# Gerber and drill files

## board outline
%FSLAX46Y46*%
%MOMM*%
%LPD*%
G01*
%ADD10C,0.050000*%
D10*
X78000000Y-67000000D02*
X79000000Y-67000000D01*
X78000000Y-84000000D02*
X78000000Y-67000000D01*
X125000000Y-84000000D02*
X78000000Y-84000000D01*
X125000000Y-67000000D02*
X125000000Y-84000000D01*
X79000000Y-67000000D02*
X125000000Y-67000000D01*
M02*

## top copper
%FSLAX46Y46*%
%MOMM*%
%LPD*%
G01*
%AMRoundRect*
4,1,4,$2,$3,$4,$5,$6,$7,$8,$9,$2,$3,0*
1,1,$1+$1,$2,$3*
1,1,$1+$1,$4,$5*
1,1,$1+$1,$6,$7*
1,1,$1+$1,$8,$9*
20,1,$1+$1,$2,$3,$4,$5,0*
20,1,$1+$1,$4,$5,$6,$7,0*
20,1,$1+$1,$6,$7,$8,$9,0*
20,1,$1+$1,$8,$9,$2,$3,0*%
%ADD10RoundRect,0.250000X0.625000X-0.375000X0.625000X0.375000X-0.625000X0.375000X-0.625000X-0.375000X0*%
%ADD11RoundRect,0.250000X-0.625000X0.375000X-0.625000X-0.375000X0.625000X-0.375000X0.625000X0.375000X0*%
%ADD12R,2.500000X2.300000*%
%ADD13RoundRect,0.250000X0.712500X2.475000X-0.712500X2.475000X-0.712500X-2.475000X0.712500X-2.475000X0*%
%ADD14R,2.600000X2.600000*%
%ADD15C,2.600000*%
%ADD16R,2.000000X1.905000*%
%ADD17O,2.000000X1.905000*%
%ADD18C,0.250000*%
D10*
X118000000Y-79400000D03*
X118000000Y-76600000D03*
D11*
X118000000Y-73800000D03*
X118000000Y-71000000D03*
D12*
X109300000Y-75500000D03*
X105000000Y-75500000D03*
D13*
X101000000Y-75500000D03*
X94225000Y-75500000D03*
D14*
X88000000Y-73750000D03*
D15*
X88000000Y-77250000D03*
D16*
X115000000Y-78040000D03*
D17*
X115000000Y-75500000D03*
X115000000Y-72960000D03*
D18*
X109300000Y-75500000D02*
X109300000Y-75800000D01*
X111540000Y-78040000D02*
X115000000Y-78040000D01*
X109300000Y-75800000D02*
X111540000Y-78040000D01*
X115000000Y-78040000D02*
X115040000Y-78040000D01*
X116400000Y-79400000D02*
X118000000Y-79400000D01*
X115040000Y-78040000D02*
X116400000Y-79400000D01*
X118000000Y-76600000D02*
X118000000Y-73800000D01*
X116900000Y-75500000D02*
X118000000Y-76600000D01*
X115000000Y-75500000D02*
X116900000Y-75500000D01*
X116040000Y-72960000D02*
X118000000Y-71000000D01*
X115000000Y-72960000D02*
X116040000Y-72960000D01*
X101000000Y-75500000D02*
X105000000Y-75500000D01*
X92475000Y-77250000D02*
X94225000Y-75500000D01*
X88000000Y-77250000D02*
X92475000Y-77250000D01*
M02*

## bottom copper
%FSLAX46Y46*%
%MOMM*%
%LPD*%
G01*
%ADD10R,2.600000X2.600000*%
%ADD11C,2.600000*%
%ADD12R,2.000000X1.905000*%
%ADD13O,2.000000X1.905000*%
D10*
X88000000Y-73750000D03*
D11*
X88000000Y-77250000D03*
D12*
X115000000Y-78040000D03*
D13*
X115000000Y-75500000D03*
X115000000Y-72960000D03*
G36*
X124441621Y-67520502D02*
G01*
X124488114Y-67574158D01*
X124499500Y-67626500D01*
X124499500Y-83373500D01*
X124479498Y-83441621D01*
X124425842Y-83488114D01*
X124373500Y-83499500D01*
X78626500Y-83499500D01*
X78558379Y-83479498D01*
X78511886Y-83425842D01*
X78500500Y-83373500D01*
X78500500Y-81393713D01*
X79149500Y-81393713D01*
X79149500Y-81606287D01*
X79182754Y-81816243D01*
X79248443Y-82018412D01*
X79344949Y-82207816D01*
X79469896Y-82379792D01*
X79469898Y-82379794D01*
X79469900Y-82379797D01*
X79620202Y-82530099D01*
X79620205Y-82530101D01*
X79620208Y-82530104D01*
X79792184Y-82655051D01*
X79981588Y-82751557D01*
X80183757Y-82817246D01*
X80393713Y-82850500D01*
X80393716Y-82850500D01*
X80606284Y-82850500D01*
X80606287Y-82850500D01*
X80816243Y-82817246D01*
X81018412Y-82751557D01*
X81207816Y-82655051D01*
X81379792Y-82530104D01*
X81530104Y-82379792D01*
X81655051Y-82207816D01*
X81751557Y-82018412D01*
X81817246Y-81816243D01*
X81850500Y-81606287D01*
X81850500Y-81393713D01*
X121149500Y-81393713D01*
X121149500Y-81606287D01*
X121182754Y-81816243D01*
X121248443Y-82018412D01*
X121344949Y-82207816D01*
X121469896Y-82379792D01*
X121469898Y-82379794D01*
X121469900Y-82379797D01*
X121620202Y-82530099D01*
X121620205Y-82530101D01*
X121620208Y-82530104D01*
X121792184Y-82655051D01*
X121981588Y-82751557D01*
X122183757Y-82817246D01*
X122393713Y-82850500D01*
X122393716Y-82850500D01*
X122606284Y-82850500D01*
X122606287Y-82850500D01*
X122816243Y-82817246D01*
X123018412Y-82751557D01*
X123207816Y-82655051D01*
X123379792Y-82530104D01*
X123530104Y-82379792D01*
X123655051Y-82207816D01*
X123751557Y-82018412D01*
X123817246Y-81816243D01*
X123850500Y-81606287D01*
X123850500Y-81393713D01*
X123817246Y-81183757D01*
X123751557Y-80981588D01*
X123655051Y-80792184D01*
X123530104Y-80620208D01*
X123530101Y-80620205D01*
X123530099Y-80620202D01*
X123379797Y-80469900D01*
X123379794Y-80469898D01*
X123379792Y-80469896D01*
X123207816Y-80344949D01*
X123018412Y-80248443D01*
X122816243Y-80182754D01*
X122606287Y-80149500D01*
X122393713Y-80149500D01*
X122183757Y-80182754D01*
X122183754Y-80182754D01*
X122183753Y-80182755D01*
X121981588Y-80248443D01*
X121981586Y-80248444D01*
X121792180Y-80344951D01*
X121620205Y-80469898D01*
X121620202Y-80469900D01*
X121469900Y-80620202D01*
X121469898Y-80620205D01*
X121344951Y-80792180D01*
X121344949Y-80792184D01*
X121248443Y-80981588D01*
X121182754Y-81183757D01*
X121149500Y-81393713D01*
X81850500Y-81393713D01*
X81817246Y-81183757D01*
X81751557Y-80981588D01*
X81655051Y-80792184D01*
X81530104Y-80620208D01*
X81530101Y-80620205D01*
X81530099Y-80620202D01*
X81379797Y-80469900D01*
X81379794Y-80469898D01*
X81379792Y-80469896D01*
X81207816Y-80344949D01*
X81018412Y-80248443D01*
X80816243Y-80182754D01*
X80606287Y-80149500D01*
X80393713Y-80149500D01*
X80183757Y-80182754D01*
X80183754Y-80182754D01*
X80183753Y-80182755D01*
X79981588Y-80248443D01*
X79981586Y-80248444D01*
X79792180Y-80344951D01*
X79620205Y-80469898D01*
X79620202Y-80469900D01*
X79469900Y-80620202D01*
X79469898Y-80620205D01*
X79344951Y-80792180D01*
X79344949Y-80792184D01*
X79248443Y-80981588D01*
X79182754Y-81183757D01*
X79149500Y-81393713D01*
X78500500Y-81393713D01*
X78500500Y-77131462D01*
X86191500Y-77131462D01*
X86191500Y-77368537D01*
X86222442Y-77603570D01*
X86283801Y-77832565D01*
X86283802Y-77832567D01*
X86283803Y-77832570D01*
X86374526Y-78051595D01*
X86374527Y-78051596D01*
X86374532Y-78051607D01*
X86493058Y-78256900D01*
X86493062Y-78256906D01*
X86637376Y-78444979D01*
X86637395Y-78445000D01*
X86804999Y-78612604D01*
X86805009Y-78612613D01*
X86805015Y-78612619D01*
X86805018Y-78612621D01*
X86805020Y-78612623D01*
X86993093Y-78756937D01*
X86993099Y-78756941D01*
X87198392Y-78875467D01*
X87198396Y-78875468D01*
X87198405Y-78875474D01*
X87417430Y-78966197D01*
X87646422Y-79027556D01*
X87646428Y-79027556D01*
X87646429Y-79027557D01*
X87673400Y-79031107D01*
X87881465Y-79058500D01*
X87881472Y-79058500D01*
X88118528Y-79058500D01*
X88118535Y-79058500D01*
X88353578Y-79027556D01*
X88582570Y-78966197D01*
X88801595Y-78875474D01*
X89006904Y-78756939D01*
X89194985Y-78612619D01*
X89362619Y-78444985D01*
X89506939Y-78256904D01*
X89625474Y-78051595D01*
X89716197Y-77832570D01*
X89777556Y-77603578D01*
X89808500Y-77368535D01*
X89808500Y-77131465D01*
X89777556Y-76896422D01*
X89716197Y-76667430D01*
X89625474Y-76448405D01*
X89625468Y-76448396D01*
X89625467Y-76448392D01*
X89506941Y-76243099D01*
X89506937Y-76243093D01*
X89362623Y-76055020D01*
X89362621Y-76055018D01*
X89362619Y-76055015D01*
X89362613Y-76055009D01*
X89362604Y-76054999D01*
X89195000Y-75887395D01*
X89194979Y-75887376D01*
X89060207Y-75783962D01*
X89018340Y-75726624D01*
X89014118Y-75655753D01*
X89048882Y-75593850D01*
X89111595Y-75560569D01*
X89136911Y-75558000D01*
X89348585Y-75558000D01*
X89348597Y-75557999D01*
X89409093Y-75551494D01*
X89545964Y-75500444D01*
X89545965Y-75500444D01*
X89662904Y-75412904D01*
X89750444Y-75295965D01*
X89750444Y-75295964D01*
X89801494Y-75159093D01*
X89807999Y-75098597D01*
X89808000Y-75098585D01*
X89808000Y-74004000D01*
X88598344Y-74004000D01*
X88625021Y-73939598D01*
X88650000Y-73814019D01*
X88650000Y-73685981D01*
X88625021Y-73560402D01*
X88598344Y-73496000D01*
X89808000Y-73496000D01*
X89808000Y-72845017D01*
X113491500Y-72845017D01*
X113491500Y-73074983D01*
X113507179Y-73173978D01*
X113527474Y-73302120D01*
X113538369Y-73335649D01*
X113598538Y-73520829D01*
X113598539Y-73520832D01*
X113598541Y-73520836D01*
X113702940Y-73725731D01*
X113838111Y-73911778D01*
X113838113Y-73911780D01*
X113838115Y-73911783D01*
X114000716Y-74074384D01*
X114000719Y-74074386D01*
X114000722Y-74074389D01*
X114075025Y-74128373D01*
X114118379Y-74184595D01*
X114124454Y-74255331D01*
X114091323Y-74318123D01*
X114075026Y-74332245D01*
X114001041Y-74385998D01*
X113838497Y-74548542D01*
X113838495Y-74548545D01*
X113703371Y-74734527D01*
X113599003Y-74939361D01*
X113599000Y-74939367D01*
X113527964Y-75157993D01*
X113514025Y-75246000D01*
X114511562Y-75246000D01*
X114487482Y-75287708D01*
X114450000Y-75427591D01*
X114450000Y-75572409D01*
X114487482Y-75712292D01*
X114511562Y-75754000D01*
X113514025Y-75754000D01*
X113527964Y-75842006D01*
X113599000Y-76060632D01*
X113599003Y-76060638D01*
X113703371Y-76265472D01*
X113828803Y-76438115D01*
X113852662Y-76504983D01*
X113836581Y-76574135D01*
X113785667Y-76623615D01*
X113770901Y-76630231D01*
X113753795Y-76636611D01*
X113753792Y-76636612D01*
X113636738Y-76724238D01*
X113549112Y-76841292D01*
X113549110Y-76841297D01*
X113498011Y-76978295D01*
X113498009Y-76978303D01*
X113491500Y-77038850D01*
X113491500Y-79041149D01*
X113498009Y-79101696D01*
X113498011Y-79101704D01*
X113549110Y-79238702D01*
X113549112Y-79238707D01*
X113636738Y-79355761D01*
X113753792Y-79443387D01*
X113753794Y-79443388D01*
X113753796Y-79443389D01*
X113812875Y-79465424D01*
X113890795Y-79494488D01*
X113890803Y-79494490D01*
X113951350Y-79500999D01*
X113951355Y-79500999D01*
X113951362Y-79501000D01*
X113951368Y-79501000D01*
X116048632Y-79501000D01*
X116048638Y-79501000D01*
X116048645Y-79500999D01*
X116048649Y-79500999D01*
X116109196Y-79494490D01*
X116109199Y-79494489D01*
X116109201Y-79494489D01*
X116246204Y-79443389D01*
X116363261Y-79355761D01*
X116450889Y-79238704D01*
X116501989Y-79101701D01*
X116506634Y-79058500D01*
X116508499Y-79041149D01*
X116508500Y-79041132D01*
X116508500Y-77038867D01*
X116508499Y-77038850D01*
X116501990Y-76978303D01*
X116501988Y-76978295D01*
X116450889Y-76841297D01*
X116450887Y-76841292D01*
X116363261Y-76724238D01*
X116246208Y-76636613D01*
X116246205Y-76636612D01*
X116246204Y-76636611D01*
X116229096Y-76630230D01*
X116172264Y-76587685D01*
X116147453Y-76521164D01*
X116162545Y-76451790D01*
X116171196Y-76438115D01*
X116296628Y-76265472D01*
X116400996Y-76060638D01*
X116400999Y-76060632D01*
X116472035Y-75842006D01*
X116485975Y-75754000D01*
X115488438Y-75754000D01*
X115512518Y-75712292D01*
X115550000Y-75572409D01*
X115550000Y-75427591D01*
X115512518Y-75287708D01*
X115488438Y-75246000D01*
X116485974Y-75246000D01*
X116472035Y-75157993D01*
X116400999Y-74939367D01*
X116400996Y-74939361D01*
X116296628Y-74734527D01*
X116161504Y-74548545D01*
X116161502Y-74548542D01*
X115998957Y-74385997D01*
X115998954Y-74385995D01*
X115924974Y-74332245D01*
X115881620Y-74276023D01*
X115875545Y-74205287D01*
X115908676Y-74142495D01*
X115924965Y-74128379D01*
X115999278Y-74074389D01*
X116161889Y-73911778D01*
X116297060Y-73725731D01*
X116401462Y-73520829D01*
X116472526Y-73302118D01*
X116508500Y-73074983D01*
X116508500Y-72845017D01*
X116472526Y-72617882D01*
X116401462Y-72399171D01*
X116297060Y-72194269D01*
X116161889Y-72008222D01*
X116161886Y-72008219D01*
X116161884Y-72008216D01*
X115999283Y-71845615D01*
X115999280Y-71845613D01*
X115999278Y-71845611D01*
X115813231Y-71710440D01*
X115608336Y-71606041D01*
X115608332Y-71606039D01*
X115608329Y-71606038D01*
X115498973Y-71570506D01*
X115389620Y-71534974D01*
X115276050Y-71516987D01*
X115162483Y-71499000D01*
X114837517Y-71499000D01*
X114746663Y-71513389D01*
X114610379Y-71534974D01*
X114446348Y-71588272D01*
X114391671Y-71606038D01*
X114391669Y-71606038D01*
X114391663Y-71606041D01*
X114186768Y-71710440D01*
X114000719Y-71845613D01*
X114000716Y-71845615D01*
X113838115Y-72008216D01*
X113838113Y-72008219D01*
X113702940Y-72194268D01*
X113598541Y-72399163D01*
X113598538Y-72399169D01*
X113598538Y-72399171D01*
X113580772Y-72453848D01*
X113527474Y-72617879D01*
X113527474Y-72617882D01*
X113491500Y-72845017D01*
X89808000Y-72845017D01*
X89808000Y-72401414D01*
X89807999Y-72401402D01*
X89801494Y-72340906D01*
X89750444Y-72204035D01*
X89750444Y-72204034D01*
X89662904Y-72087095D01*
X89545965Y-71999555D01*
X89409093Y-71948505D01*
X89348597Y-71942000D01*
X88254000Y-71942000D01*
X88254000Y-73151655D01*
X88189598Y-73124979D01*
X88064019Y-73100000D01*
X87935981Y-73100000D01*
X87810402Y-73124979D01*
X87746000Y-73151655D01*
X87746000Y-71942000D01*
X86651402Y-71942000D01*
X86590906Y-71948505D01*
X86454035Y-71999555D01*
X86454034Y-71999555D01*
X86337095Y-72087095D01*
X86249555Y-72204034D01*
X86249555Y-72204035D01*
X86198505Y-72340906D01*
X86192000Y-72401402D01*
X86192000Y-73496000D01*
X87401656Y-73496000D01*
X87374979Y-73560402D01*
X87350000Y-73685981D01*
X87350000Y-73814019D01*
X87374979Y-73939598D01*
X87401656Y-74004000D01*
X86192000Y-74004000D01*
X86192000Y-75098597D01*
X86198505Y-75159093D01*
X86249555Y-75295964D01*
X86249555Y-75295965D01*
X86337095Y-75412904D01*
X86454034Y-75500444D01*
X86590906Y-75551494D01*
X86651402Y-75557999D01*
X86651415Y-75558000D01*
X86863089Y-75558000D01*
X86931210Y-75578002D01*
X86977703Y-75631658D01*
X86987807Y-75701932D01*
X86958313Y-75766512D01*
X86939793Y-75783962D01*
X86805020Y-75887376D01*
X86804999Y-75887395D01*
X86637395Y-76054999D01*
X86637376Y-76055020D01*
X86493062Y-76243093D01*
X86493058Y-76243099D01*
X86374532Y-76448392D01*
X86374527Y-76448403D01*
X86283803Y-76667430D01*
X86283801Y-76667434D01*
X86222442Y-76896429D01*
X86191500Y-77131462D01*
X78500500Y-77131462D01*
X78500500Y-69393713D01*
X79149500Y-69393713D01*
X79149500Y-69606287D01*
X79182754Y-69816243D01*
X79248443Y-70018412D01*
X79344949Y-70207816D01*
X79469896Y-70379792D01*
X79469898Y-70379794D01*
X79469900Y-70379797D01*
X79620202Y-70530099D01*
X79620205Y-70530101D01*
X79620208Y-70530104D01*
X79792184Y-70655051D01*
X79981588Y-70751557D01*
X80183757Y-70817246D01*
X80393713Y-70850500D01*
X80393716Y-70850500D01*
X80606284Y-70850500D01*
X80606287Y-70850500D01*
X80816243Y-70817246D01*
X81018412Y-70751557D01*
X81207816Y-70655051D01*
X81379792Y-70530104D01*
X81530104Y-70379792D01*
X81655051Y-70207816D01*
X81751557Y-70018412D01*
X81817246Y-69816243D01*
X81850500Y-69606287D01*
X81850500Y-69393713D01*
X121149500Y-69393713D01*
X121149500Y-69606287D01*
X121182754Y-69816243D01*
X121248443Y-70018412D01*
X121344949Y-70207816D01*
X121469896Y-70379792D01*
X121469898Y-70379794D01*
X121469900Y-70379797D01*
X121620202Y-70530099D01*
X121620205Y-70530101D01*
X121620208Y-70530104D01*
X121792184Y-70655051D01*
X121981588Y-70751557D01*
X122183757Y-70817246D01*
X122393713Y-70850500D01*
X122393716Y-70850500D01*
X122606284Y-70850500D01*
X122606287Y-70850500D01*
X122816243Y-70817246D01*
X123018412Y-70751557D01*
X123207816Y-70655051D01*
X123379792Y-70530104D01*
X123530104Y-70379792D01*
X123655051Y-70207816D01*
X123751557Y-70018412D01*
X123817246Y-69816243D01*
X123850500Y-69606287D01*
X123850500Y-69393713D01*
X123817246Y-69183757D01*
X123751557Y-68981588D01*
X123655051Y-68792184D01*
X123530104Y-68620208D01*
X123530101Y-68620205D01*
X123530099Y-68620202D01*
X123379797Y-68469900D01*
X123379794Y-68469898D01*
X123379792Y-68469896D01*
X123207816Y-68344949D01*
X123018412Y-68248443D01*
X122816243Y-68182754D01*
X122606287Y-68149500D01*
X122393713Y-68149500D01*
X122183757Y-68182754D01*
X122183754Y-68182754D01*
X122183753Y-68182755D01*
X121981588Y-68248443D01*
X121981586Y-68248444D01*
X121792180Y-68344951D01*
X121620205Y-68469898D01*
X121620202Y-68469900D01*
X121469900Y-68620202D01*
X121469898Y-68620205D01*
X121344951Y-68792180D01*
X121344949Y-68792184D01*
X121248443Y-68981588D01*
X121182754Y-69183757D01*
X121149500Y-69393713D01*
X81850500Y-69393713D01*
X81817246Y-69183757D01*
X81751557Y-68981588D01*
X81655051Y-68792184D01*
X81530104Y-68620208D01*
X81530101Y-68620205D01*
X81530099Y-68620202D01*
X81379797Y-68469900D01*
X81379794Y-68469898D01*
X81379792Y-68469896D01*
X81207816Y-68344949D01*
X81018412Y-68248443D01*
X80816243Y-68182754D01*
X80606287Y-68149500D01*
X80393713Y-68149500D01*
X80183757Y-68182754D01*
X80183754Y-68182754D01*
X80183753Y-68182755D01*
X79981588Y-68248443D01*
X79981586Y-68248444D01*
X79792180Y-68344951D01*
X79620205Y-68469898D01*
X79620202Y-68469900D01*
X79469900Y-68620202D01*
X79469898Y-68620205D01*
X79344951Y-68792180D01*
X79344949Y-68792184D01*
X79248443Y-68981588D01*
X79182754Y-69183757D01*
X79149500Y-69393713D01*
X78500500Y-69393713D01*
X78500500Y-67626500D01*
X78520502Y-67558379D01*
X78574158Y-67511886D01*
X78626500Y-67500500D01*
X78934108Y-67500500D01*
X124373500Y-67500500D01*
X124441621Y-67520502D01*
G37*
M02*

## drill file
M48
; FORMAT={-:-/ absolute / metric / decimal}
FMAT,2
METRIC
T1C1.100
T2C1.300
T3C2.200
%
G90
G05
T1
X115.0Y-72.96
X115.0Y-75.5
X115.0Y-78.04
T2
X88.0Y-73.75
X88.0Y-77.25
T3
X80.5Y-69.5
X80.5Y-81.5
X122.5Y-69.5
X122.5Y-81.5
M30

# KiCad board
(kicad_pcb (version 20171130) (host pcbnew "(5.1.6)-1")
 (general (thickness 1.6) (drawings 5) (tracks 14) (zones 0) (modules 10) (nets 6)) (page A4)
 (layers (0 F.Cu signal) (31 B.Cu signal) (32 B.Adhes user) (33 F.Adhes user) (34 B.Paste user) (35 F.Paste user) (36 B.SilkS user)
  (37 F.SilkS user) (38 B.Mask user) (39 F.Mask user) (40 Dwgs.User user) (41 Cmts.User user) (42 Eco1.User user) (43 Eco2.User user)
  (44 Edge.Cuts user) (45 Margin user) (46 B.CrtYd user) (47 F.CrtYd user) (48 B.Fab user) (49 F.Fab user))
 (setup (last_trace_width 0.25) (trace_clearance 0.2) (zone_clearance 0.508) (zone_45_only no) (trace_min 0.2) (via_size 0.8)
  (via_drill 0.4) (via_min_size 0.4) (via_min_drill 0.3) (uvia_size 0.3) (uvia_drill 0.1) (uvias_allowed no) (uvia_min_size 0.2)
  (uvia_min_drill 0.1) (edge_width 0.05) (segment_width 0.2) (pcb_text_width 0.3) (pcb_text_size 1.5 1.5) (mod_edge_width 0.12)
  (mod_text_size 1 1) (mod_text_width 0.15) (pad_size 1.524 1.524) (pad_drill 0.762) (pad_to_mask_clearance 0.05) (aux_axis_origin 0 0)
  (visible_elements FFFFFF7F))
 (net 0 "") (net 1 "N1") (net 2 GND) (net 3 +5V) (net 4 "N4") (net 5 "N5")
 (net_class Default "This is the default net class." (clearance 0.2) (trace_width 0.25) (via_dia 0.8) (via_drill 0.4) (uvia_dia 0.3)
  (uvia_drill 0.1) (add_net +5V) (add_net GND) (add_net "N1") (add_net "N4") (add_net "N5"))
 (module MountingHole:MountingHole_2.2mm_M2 (layer F.Cu) (at 80.5 69.5)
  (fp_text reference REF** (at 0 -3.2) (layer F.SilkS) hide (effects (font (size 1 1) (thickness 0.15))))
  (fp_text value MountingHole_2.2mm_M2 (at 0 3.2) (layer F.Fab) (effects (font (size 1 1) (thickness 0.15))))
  (pad 1 np_thru_hole circle (at 0 0) (size 2.2 2.2) (drill 2.2) (layers *.Cu *.Mask)))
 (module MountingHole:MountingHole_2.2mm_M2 (layer F.Cu) (at 80.5 81.5)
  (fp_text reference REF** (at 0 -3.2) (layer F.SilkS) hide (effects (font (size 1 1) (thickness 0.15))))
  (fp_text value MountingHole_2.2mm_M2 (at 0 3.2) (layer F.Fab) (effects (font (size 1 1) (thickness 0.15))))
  (pad 1 np_thru_hole circle (at 0 0) (size 2.2 2.2) (drill 2.2) (layers *.Cu *.Mask)))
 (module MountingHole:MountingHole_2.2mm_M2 (layer F.Cu) (at 122.5 81.5)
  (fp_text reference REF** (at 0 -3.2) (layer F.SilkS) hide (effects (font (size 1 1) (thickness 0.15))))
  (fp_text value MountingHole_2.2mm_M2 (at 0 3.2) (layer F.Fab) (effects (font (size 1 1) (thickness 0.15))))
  (pad 1 np_thru_hole circle (at 0 0) (size 2.2 2.2) (drill 2.2) (layers *.Cu *.Mask)))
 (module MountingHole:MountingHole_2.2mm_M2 (layer F.Cu) (at 122.5 69.5)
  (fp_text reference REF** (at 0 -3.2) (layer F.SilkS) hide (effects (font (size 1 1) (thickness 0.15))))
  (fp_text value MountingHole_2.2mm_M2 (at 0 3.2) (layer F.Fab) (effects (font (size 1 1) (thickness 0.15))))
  (pad 1 np_thru_hole circle (at 0 0) (size 2.2 2.2) (drill 2.2) (layers *.Cu *.Mask)))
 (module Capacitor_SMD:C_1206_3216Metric (layer F.Cu) (at 118 78 90)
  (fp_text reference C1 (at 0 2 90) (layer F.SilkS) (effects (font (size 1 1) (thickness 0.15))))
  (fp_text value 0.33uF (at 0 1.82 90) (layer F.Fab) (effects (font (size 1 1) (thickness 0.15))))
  (pad 1 smd roundrect (at -1.4 0 90) (size 1.25 1.75) (layers F.Cu F.Paste F.Mask) (roundrect_rratio 0.2) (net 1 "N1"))
  (pad 2 smd roundrect (at 1.4 0 90) (size 1.25 1.75) (layers F.Cu F.Paste F.Mask) (roundrect_rratio 0.2) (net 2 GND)))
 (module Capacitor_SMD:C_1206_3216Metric (layer F.Cu) (at 118 72.4 270)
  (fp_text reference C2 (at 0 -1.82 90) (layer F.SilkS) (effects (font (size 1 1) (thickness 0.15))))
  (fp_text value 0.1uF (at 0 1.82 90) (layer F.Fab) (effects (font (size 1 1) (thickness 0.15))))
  (pad 2 smd roundrect (at 1.4 0 270) (size 1.25 1.75) (layers F.Cu F.Paste F.Mask) (roundrect_rratio 0.2) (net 2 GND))
  (pad 1 smd roundrect (at -1.4 0 270) (size 1.25 1.75) (layers F.Cu F.Paste F.Mask) (roundrect_rratio 0.2) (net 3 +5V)))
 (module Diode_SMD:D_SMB (layer F.Cu) (at 107.15 75.5 180)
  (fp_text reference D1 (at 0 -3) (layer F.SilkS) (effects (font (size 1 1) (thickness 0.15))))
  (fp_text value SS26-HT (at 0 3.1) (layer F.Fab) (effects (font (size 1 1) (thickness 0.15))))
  (pad 1 smd rect (at -2.15 0 180) (size 2.5 2.3) (layers F.Cu F.Paste F.Mask) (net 1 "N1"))
  (pad 2 smd rect (at 2.15 0 180) (size 2.5 2.3) (layers F.Cu F.Paste F.Mask) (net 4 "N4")))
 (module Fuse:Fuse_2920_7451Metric (layer F.Cu) (at 97.6125 75.5 180)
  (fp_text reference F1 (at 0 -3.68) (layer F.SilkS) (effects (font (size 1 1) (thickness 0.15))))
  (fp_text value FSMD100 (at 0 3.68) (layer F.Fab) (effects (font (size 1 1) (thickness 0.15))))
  (pad 1 smd roundrect (at -3.3875 0 180) (size 1.925 5.45) (layers F.Cu F.Paste F.Mask) (roundrect_rratio 0.12987) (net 4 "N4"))
  (pad 2 smd roundrect (at 3.3875 0 180) (size 1.925 5.45) (layers F.Cu F.Paste F.Mask) (roundrect_rratio 0.12987) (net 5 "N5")))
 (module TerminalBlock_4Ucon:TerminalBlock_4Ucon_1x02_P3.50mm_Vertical (layer F.Cu) (at 88 73.75 270)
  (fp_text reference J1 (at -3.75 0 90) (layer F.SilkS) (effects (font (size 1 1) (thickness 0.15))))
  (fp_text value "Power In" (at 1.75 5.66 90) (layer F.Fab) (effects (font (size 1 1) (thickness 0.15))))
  (pad 1 thru_hole rect (at 0 0 270) (size 2.6 2.6) (drill 1.3) (layers *.Cu *.Mask) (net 2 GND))
  (pad 2 thru_hole circle (at 3.5 0 270) (size 2.6 2.6) (drill 1.3) (layers *.Cu *.Mask) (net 5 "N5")))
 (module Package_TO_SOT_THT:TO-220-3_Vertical (layer F.Cu) (at 115 78.04 90)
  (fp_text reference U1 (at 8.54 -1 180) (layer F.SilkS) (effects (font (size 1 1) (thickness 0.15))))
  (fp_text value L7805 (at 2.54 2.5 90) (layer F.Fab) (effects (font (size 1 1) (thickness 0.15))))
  (pad 1 thru_hole rect (at 0 0 90) (size 1.905 2) (drill 1.1) (layers *.Cu *.Mask) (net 1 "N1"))
  (pad 2 thru_hole oval (at 2.54 0 90) (size 1.905 2) (drill 1.1) (layers *.Cu *.Mask) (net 2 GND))
  (pad 3 thru_hole oval (at 5.08 0 90) (size 1.905 2) (drill 1.1) (layers *.Cu *.Mask) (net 3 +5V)))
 (gr_line (start 78 67) (end 79 67) (layer Edge.Cuts) (width 0.05))
 (gr_line (start 78 84) (end 78 67) (layer Edge.Cuts) (width 0.05))
 (gr_line (start 125 84) (end 78 84) (layer Edge.Cuts) (width 0.05))
 (gr_line (start 125 67) (end 125 84) (layer Edge.Cuts) (width 0.05))
 (gr_line (start 79 67) (end 125 67) (layer Edge.Cuts) (width 0.05))
 (segment (start 109.3 75.5) (end 109.3 75.8) (width 0.25) (layer F.Cu) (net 1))
 (segment (start 111.54 78.04) (end 115 78.04) (width 0.25) (layer F.Cu) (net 1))
 (segment (start 109.3 75.8) (end 111.54 78.04) (width 0.25) (layer F.Cu) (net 1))
 (segment (start 115 78.04) (end 115.04 78.04) (width 0.25) (layer F.Cu) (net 1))
 (segment (start 116.4 79.4) (end 118 79.4) (width 0.25) (layer F.Cu) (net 1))
 (segment (start 115.04 78.04) (end 116.4 79.4) (width 0.25) (layer F.Cu) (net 1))
 (segment (start 118 76.6) (end 118 73.8) (width 0.25) (layer F.Cu) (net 2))
 (segment (start 116.9 75.5) (end 118 76.6) (width 0.25) (layer F.Cu) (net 2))
 (segment (start 115 75.5) (end 116.9 75.5) (width 0.25) (layer F.Cu) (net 2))
 (segment (start 116.04 72.96) (end 118 71) (width 0.25) (layer F.Cu) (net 3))
 (segment (start 115 72.96) (end 116.04 72.96) (width 0.25) (layer F.Cu) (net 3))
 (segment (start 101 75.5) (end 105 75.5) (width 0.25) (layer F.Cu) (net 4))
 (segment (start 92.475 77.25) (end 94.225 75.5) (width 0.25) (layer F.Cu) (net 5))
 (segment (start 88 77.25) (end 92.475 77.25) (width 0.25) (layer F.Cu) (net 5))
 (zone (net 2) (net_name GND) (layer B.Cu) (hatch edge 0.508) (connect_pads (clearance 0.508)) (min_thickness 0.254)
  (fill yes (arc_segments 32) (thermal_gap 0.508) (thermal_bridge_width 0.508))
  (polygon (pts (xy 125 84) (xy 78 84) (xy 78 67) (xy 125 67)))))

